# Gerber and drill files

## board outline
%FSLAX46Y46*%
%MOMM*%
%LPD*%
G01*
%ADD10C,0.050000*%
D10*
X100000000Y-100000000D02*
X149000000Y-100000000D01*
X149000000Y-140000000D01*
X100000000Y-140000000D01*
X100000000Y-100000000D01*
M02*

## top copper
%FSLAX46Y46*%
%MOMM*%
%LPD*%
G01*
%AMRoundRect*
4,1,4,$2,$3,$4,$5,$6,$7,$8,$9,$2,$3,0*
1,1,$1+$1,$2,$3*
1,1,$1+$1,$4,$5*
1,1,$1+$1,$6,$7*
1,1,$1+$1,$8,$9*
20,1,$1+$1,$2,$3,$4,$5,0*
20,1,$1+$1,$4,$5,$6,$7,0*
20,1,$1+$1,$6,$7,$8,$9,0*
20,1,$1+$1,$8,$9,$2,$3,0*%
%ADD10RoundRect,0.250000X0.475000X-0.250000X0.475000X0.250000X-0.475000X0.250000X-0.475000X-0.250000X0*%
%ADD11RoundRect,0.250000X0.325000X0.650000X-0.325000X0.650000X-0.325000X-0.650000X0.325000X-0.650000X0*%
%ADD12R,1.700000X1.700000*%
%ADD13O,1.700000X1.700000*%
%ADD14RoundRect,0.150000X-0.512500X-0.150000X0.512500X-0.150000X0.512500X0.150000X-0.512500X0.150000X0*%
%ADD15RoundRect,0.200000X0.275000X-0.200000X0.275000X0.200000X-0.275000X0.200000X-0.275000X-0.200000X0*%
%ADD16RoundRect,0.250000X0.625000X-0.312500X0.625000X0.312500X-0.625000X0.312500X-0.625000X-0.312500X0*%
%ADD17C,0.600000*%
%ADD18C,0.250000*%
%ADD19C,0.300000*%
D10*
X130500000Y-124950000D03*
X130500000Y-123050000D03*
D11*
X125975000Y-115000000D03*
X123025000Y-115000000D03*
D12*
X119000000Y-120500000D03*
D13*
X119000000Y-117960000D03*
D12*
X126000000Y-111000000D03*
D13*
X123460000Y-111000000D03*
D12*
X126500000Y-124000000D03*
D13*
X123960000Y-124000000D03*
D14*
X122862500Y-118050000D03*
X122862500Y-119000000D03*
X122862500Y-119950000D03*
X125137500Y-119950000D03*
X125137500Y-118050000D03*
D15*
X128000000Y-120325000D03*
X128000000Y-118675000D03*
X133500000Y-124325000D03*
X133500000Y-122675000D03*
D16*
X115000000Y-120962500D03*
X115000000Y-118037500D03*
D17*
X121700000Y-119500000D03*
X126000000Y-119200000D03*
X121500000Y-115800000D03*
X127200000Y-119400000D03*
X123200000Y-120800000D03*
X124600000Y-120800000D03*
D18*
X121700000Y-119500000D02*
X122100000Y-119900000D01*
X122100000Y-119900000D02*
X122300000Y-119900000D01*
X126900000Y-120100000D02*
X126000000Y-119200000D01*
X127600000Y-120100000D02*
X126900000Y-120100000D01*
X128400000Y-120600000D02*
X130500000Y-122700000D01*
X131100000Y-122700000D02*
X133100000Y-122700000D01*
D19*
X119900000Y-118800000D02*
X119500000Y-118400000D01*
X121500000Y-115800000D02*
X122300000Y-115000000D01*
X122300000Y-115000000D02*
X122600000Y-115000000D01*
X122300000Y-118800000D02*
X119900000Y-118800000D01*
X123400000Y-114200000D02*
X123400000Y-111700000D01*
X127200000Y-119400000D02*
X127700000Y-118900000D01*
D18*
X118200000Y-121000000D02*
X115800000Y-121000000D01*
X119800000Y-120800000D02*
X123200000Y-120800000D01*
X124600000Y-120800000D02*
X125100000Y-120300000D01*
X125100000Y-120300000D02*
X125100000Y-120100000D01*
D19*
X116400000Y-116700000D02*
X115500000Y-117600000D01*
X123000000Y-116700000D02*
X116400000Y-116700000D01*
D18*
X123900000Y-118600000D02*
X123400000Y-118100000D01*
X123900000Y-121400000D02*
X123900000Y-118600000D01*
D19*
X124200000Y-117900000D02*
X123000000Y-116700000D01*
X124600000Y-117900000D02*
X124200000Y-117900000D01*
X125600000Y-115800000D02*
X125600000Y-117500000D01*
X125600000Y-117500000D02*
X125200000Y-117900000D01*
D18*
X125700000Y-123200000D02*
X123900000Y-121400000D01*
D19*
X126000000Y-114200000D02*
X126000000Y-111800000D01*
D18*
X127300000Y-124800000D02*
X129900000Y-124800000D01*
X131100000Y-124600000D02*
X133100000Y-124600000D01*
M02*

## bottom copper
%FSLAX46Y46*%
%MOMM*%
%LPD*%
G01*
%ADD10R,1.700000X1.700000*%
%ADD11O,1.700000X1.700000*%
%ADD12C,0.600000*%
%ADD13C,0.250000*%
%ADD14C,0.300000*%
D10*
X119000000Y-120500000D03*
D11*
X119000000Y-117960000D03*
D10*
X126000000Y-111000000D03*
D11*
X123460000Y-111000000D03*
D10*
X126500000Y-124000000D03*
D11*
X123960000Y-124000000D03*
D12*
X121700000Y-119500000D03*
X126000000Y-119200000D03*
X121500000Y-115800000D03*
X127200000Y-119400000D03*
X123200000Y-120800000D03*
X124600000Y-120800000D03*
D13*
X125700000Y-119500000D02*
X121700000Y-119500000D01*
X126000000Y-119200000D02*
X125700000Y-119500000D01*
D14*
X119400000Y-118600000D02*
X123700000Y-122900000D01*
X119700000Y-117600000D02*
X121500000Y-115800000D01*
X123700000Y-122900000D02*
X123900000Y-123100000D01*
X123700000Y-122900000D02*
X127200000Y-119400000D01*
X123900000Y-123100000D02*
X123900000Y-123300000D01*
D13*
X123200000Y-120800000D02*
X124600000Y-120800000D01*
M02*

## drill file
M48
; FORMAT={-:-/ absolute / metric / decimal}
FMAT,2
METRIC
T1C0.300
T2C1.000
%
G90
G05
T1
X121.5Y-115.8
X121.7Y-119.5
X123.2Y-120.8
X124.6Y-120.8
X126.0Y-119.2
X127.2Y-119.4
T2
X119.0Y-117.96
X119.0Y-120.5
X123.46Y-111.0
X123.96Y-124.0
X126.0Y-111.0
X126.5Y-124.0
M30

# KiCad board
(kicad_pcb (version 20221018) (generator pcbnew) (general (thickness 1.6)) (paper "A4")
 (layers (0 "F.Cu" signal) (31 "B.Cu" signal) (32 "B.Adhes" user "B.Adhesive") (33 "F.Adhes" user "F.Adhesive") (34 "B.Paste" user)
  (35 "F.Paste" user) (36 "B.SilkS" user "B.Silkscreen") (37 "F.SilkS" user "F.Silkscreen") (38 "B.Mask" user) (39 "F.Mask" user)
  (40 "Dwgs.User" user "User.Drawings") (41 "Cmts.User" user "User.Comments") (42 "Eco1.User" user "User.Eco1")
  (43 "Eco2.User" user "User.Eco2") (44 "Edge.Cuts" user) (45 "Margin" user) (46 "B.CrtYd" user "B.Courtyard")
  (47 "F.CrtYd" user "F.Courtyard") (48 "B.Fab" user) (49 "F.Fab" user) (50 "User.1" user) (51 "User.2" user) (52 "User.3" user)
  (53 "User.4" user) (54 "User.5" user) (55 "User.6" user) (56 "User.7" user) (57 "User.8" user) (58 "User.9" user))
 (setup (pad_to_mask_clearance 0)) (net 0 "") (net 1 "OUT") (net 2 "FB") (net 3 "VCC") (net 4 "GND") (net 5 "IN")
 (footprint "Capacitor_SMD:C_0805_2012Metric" (layer "F.Cu") (at 130.5 124 90)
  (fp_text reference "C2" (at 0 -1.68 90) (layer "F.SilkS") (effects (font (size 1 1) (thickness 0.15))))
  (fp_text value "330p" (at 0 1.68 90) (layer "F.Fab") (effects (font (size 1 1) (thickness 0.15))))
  (pad "1" smd roundrect (at -0.95 0 90) (size 1 1.45) (layers "F.Cu" "F.Paste" "F.Mask") (roundrect_rratio 0.25) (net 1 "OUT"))
  (pad "2" smd roundrect (at 0.95 0 90) (size 1 1.45) (layers "F.Cu" "F.Paste" "F.Mask") (roundrect_rratio 0.25) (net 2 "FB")))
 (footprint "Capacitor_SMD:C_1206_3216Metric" (layer "F.Cu") (at 124.5 115 180)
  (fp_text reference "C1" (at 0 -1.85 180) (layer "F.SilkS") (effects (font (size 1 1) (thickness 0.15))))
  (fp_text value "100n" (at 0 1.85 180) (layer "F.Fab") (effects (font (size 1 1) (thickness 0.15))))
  (pad "1" smd roundrect (at -1.475 0 180) (size 1.15 1.8) (layers "F.Cu" "F.Paste" "F.Mask") (roundrect_rratio 0.217391) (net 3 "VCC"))
  (pad "2" smd roundrect (at 1.475 0 180) (size 1.15 1.8) (layers "F.Cu" "F.Paste" "F.Mask") (roundrect_rratio 0.217391) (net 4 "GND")))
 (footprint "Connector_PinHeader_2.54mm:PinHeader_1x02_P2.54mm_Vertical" (layer "F.Cu") (at 119 120.5 180)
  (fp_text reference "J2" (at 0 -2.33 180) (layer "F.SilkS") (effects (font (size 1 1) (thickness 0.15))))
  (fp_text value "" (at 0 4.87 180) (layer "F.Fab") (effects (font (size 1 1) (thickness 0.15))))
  (pad "1" thru_hole rect (at 0 0 180) (size 1.7 1.7) (drill 1) (layers "*.Cu" "*.Mask") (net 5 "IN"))
  (pad "2" thru_hole oval (at 0 2.54 180) (size 1.7 1.7) (drill 1) (layers "*.Cu" "*.Mask") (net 4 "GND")))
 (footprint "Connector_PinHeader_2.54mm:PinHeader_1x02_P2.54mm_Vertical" (layer "F.Cu") (at 126 111 -90)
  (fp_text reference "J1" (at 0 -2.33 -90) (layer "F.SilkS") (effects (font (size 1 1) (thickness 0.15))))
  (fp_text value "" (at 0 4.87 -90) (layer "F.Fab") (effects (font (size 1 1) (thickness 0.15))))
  (pad "1" thru_hole rect (at 0 0 270) (size 1.7 1.7) (drill 1) (layers "*.Cu" "*.Mask") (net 3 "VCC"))
  (pad "2" thru_hole oval (at 0 2.54 270) (size 1.7 1.7) (drill 1) (layers "*.Cu" "*.Mask") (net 4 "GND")))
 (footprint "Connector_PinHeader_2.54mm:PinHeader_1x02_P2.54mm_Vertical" (layer "F.Cu") (at 126.5 124 -90)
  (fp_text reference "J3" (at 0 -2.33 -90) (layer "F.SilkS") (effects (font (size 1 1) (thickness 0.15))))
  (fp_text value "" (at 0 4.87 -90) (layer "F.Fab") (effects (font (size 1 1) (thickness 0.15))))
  (pad "1" thru_hole rect (at 0 0 270) (size 1.7 1.7) (drill 1) (layers "*.Cu" "*.Mask") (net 1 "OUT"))
  (pad "2" thru_hole oval (at 0 2.54 270) (size 1.7 1.7) (drill 1) (layers "*.Cu" "*.Mask") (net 4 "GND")))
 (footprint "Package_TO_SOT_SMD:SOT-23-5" (layer "F.Cu") (at 124 119)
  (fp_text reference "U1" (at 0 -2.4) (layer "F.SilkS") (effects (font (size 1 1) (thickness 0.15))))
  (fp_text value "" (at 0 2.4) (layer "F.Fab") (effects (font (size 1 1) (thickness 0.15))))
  (pad "1" smd roundrect (at -1.1375 -0.95) (size 1.325 0.6) (layers "F.Cu" "F.Paste" "F.Mask") (roundrect_rratio 0.25) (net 1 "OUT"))
  (pad "2" smd roundrect (at -1.1375 0) (size 1.325 0.6) (layers "F.Cu" "F.Paste" "F.Mask") (roundrect_rratio 0.25) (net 4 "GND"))
  (pad "3" smd roundrect (at -1.1375 0.95) (size 1.325 0.6) (layers "F.Cu" "F.Paste" "F.Mask") (roundrect_rratio 0.25) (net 2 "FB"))
  (pad "4" smd roundrect (at 1.1375 0.95) (size 1.325 0.6) (layers "F.Cu" "F.Paste" "F.Mask") (roundrect_rratio 0.25) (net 5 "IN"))
  (pad "5" smd roundrect (at 1.1375 -0.95) (size 1.325 0.6) (layers "F.Cu" "F.Paste" "F.Mask") (roundrect_rratio 0.25) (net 3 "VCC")))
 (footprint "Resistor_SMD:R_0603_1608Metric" (layer "F.Cu") (at 128 119.5 90)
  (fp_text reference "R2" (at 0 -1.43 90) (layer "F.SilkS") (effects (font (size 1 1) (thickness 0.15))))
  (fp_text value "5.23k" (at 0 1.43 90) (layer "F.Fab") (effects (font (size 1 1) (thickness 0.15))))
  (pad "1" smd roundrect (at -0.825 0 90) (size 0.8 0.95) (layers "F.Cu" "F.Paste" "F.Mask") (roundrect_rratio 0.25) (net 2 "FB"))
  (pad "2" smd roundrect (at 0.825 0 90) (size 0.8 0.95) (layers "F.Cu" "F.Paste" "F.Mask") (roundrect_rratio 0.25) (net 4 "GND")))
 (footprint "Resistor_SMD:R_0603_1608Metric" (layer "F.Cu") (at 133.5 123.5 90)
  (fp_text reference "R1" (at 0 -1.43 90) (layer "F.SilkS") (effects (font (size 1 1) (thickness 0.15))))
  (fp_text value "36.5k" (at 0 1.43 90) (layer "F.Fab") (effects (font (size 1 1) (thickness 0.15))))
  (pad "1" smd roundrect (at -0.825 0 90) (size 0.8 0.95) (layers "F.Cu" "F.Paste" "F.Mask") (roundrect_rratio 0.25) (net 1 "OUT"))
  (pad "2" smd roundrect (at 0.825 0 90) (size 0.8 0.95) (layers "F.Cu" "F.Paste" "F.Mask") (roundrect_rratio 0.25) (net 2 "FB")))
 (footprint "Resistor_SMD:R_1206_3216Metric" (layer "F.Cu") (at 115 119.5 90)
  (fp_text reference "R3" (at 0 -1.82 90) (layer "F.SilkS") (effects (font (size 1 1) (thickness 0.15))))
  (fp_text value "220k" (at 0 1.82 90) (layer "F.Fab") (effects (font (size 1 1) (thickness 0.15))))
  (pad "1" smd roundrect (at -1.4625 0 90) (size 1.125 1.75) (layers "F.Cu" "F.Paste" "F.Mask") (roundrect_rratio 0.222222) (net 5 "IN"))
  (pad "2" smd roundrect (at 1.4625 0 90) (size 1.125 1.75) (layers "F.Cu" "F.Paste" "F.Mask") (roundrect_rratio 0.222222) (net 3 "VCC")))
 (gr_rect (start 100 100) (end 149 140) (stroke (width 0.05) (type default)) (fill none) (layer "Edge.Cuts"))
 (segment (start 121.7 119.5) (end 122.1 119.9) (width 0.25) (layer "F.Cu") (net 2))
 (segment (start 122.1 119.9) (end 122.3 119.9) (width 0.25) (layer "F.Cu") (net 2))
 (segment (start 126.9 120.1) (end 126 119.2) (width 0.25) (layer "F.Cu") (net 2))
 (segment (start 127.6 120.1) (end 126.9 120.1) (width 0.25) (layer "F.Cu") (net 2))
 (segment (start 128.4 120.6) (end 130.5 122.7) (width 0.25) (layer "F.Cu") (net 2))
 (segment (start 131.1 122.7) (end 133.1 122.7) (width 0.25) (layer "F.Cu") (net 2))
 (via (at 121.7 119.5) (size 0.6) (drill 0.3) (layers "F.Cu" "B.Cu") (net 2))
 (via (at 126 119.2) (size 0.6) (drill 0.3) (layers "F.Cu" "B.Cu") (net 2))
 (segment (start 119.9 118.8) (end 119.5 118.4) (width 0.3) (layer "F.Cu") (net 4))
 (segment (start 121.5 115.8) (end 122.3 115) (width 0.3) (layer "F.Cu") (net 4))
 (segment (start 122.3 115) (end 122.6 115) (width 0.3) (layer "F.Cu") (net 4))
 (segment (start 122.3 118.8) (end 119.9 118.8) (width 0.3) (layer "F.Cu") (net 4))
 (segment (start 123.4 114.2) (end 123.4 111.7) (width 0.3) (layer "F.Cu") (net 4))
 (segment (start 125.7 119.5) (end 121.7 119.5) (width 0.25) (layer "B.Cu") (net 2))
 (segment (start 126 119.2) (end 125.7 119.5) (width 0.25) (layer "B.Cu") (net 2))
 (segment (start 127.2 119.4) (end 127.7 118.9) (width 0.3) (layer "F.Cu") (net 4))
 (via (at 121.5 115.8) (size 0.6) (drill 0.3) (layers "F.Cu" "B.Cu") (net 4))
 (via (at 127.2 119.4) (size 0.6) (drill 0.3) (layers "F.Cu" "B.Cu") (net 4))
 (segment (start 118.2 121) (end 115.8 121) (width 0.25) (layer "F.Cu") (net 5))
 (segment (start 119.4 118.6) (end 123.7 122.9) (width 0.3) (layer "B.Cu") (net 4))
 (segment (start 119.7 117.6) (end 121.5 115.8) (width 0.3) (layer "B.Cu") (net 4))
 (segment (start 119.8 120.8) (end 123.2 120.8) (width 0.25) (layer "F.Cu") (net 5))
 (segment (start 123.7 122.9) (end 123.9 123.1) (width 0.3) (layer "B.Cu") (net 4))
 (segment (start 123.7 122.9) (end 127.2 119.4) (width 0.3) (layer "B.Cu") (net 4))
 (segment (start 123.9 123.1) (end 123.9 123.3) (width 0.3) (layer "B.Cu") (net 4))
 (segment (start 124.6 120.8) (end 125.1 120.3) (width 0.25) (layer "F.Cu") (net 5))
 (segment (start 125.1 120.3) (end 125.1 120.1) (width 0.25) (layer "F.Cu") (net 5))
 (via (at 123.2 120.8) (size 0.6) (drill 0.3) (layers "F.Cu" "B.Cu") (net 5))
 (via (at 124.6 120.8) (size 0.6) (drill 0.3) (layers "F.Cu" "B.Cu") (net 5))
 (segment (start 116.4 116.7) (end 115.5 117.6) (width 0.3) (layer "F.Cu") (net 3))
 (segment (start 123 116.7) (end 116.4 116.7) (width 0.3) (layer "F.Cu") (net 3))
 (segment (start 123.2 120.8) (end 124.6 120.8) (width 0.25) (layer "B.Cu") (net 5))
 (segment (start 123.9 118.6) (end 123.4 118.1) (width 0.25) (layer "F.Cu") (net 1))
 (segment (start 123.9 121.4) (end 123.9 118.6) (width 0.25) (layer "F.Cu") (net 1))
 (segment (start 124.2 117.9) (end 123 116.7) (width 0.3) (layer "F.Cu") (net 3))
 (segment (start 124.6 117.9) (end 124.2 117.9) (width 0.3) (layer "F.Cu") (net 3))
 (segment (start 125.6 115.8) (end 125.6 117.5) (width 0.3) (layer "F.Cu") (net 3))
 (segment (start 125.6 117.5) (end 125.2 117.9) (width 0.3) (layer "F.Cu") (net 3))
 (segment (start 125.7 123.2) (end 123.9 121.4) (width 0.25) (layer "F.Cu") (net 1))
 (segment (start 126 114.2) (end 126 111.8) (width 0.3) (layer "F.Cu") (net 3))
 (segment (start 127.3 124.8) (end 129.9 124.8) (width 0.25) (layer "F.Cu") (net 1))
 (segment (start 131.1 124.6) (end 133.1 124.6) (width 0.25) (layer "F.Cu") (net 1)))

